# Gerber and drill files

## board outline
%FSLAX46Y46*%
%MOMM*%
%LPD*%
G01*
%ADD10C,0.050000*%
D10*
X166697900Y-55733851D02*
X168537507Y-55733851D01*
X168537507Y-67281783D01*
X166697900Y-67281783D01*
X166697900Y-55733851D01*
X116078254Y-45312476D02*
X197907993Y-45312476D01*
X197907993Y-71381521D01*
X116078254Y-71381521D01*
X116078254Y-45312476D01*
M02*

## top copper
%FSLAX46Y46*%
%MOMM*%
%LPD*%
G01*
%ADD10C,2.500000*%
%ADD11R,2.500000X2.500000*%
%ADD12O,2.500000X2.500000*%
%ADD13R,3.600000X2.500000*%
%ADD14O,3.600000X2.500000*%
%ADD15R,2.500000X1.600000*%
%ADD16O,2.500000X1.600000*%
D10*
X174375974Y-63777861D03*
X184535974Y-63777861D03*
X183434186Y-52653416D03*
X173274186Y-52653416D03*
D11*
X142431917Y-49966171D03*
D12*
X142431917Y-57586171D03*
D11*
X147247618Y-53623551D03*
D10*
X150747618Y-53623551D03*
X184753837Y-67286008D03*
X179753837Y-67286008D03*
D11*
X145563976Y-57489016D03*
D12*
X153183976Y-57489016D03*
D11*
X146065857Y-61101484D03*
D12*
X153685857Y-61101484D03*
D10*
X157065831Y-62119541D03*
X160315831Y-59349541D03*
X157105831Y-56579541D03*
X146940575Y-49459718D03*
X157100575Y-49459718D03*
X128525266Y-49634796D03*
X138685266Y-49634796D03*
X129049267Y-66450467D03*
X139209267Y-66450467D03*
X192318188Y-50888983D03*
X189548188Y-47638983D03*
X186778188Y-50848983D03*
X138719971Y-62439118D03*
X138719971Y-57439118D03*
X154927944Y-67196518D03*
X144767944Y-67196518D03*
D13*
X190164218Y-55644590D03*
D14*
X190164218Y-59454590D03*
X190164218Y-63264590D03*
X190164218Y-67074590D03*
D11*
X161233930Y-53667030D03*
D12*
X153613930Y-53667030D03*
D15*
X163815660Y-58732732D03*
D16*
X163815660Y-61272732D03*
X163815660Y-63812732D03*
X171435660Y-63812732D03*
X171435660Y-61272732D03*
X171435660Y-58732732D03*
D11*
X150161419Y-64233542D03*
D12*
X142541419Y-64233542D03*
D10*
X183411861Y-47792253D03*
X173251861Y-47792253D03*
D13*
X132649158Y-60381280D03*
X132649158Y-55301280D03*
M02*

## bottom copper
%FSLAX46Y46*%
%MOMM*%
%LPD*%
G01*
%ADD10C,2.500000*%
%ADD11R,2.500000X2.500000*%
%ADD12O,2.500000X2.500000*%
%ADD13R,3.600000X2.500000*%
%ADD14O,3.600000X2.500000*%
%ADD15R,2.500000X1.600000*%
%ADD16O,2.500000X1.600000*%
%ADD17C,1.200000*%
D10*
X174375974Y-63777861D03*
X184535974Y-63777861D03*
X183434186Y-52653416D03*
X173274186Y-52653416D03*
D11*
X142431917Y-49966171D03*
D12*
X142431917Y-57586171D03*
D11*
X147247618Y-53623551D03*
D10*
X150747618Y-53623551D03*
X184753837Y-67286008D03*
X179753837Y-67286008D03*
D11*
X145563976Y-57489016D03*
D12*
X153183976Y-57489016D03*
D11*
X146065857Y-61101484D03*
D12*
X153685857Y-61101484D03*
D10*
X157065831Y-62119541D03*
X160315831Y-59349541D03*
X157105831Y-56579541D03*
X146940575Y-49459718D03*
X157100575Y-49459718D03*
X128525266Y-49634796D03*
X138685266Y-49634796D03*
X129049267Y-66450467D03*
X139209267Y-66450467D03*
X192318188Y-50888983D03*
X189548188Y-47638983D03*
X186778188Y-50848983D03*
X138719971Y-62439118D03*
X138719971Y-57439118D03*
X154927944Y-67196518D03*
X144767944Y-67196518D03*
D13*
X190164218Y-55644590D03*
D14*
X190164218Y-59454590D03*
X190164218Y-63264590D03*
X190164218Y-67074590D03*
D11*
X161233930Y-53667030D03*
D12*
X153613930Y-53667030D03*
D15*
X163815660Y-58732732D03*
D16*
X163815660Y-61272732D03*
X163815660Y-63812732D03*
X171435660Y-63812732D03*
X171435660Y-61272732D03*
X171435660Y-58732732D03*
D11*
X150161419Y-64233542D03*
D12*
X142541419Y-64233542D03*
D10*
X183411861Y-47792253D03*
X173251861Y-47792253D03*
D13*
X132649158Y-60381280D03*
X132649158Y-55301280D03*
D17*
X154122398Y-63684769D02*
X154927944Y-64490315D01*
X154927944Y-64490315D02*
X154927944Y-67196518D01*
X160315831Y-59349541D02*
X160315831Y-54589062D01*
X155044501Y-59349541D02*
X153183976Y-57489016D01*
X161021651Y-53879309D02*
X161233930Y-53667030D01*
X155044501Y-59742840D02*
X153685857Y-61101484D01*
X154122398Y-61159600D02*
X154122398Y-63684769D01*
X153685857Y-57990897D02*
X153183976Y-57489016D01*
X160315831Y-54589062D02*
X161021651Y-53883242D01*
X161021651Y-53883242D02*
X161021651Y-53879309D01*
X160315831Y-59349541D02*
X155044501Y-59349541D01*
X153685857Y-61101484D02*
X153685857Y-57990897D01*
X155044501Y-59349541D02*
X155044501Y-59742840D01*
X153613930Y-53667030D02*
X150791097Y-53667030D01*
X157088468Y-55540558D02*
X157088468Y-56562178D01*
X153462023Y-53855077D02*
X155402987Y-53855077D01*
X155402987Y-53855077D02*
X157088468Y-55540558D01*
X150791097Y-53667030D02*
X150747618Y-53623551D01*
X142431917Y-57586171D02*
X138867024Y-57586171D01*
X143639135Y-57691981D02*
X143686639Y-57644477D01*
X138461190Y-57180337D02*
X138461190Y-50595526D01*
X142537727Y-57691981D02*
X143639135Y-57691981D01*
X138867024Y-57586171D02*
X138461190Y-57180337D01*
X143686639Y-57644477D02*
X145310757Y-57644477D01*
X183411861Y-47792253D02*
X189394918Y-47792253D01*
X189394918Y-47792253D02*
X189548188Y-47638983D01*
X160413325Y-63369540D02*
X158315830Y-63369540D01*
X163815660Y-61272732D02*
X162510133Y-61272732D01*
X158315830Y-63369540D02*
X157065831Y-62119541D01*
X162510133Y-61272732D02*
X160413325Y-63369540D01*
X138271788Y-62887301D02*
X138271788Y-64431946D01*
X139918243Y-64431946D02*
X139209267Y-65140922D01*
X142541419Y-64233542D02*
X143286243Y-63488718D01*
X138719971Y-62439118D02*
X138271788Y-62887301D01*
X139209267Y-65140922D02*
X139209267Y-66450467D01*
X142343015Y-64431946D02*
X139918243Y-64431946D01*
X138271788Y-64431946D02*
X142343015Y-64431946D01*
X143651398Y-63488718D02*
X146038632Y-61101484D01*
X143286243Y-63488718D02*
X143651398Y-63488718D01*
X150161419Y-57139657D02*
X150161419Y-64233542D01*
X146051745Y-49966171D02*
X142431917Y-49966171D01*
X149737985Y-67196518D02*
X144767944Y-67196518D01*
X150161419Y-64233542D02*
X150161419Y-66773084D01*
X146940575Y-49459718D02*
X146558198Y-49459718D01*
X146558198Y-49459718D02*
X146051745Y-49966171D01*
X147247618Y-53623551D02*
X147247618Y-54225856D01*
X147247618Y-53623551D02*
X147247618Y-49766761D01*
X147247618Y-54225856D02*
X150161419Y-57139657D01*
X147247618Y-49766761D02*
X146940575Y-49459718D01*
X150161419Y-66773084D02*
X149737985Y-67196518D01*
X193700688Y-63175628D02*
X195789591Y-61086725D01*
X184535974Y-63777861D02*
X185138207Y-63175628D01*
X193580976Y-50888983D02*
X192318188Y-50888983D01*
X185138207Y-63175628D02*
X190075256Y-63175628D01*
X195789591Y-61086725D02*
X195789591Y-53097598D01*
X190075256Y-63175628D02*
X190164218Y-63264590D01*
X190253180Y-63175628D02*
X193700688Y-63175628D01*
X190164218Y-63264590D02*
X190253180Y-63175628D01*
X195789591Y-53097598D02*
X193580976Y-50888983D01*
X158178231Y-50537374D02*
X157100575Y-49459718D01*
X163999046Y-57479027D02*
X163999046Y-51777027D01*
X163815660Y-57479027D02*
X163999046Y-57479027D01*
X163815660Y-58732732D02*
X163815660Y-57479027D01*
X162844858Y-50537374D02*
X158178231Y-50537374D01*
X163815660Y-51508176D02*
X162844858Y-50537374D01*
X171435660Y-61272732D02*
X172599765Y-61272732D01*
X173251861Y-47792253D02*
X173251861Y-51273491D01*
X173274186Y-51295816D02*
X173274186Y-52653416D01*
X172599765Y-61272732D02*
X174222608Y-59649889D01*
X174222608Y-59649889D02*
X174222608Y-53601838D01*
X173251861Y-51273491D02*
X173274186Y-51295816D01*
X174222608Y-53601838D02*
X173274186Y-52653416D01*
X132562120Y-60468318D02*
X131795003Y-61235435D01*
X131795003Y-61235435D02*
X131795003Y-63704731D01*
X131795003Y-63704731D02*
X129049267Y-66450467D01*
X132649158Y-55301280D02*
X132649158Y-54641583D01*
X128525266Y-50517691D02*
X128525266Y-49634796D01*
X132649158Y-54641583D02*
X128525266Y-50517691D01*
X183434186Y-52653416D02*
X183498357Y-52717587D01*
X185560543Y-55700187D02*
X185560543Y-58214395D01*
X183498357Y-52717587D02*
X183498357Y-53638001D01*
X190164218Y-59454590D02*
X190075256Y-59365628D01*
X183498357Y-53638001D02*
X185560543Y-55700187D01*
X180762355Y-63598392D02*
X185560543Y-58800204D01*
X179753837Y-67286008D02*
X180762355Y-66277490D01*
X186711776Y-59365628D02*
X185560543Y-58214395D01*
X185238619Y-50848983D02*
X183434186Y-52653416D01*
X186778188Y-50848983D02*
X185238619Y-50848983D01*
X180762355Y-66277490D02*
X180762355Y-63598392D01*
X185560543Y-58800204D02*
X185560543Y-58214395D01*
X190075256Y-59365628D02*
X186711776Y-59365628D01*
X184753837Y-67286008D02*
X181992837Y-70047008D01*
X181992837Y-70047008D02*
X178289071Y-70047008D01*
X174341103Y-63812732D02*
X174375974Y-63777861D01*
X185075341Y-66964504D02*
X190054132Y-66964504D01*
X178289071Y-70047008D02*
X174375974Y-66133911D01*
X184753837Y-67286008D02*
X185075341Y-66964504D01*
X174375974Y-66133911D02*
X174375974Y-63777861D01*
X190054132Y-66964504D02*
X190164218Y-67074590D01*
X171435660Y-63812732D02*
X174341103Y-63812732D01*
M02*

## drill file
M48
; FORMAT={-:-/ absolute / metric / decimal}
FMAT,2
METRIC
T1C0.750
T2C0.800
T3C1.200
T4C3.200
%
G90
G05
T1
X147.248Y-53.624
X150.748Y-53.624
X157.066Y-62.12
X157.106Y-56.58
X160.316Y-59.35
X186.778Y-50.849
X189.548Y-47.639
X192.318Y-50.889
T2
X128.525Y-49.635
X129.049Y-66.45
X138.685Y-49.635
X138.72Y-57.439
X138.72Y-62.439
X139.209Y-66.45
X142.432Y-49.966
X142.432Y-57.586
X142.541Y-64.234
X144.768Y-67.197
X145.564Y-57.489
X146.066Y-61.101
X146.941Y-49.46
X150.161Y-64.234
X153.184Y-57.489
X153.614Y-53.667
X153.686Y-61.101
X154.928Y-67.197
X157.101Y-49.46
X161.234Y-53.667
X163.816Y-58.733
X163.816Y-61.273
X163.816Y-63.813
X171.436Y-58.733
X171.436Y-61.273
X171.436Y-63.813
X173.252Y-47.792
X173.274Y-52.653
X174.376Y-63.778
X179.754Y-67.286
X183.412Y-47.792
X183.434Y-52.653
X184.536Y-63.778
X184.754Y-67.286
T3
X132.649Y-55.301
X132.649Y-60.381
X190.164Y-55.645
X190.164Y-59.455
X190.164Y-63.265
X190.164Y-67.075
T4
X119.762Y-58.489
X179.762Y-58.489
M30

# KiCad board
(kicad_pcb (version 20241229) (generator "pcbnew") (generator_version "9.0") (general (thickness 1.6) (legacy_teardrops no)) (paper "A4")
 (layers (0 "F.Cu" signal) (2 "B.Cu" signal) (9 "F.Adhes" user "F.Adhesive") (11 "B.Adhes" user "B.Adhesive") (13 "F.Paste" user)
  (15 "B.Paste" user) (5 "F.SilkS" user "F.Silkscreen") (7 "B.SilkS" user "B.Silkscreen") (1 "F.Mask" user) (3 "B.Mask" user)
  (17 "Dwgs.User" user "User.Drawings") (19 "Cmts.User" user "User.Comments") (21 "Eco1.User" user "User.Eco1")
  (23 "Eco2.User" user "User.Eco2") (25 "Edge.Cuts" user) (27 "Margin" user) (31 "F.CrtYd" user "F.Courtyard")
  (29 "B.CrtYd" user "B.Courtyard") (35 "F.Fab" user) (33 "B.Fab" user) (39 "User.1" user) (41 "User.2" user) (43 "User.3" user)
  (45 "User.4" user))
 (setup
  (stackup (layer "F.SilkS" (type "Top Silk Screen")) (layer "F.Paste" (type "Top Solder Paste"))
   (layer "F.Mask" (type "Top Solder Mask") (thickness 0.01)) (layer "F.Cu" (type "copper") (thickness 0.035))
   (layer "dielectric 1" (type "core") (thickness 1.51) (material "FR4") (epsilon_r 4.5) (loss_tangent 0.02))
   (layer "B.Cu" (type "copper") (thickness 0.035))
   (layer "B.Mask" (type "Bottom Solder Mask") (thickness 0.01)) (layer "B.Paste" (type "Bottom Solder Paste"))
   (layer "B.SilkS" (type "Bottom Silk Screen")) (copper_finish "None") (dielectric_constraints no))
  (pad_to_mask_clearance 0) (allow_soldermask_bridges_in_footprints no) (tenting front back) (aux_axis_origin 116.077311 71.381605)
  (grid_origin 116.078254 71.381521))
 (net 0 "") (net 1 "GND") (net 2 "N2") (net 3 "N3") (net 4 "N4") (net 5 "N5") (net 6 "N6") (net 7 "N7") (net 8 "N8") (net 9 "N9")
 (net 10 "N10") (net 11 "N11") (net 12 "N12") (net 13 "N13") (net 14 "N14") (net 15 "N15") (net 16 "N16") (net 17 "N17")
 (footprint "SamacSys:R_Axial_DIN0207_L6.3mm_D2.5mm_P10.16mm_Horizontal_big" (layer "F.Cu") (at 174.375974 63.777861)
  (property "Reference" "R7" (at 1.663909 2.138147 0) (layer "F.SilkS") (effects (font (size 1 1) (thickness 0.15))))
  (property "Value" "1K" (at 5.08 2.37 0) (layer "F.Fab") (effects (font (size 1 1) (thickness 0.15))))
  (pad "1" thru_hole circle (at 0 0) (size 2.5 2.5) (drill 0.8) (layers "*.Cu" "*.Mask") (remove_unused_layers no) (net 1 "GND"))
  (pad "2" thru_hole circle (at 10.16 0) (size 2.5 2.5) (drill 0.8) (layers "*.Cu" "*.Mask") (remove_unused_layers no) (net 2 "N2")))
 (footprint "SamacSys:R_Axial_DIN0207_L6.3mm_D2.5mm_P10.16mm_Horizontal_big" (layer "F.Cu") (at 183.434186 52.653416 180)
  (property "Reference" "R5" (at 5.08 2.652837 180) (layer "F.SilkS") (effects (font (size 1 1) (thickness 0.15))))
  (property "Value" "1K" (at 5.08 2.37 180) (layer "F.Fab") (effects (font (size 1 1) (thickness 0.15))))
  (pad "1" thru_hole circle (at 0 0 180) (size 2.5 2.5) (drill 0.8) (layers "*.Cu" "*.Mask") (remove_unused_layers no) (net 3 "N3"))
  (pad "2" thru_hole circle (at 10.16 0 180) (size 2.5 2.5) (drill 0.8) (layers "*.Cu" "*.Mask") (remove_unused_layers no) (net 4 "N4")))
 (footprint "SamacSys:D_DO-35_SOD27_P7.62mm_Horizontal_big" (layer "F.Cu") (at 142.431917 49.966171 -90)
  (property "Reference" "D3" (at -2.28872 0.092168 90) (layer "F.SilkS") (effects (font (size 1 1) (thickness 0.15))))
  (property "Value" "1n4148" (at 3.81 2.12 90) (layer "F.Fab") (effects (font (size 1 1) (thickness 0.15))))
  (pad "1" thru_hole rect (at 0 0 270) (size 2.5 2.5) (drill 0.8) (layers "*.Cu" "*.Mask") (remove_unused_layers no) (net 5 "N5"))
  (pad "2" thru_hole oval (at 7.62 0 270) (size 2.5 2.5) (drill 0.8) (layers "*.Cu" "*.Mask") (remove_unused_layers no) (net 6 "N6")))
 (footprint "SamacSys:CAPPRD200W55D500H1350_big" (layer "F.Cu") (at 147.247618 53.623551)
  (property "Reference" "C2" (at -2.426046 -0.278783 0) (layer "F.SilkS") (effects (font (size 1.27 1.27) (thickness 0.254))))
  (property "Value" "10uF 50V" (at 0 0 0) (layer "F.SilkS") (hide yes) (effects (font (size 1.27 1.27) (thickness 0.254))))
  (pad "1" thru_hole rect (at 0 0) (size 2.5 2.5) (drill 0.75) (layers "*.Cu" "*.Mask") (remove_unused_layers no) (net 5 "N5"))
  (pad "2" thru_hole circle (at 3.5 0) (size 2.5 2.5) (drill 0.75) (layers "*.Cu" "*.Mask") (remove_unused_layers no) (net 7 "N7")))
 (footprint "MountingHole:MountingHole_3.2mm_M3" (layer "F.Cu") (at 179.762141 58.489223)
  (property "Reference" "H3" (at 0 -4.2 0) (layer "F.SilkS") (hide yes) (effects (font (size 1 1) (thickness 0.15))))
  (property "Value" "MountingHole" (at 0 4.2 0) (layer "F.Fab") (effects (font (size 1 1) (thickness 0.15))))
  (pad "" np_thru_hole circle (at 0 0) (size 3.2 3.2) (drill 3.2) (layers "*.Cu" "*.Mask")))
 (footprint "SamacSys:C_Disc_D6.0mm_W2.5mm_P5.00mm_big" (layer "F.Cu") (at 184.753837 67.286008 180)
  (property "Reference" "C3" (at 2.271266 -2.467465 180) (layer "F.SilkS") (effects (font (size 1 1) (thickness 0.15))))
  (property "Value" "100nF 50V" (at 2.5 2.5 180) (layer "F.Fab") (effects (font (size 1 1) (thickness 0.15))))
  (pad "1" thru_hole circle (at 0 0 180) (size 2.5 2.5) (drill 0.8) (layers "*.Cu" "*.Mask") (remove_unused_layers no) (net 1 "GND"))
  (pad "2" thru_hole circle (at 5 0 180) (size 2.5 2.5) (drill 0.8) (layers "*.Cu" "*.Mask") (remove_unused_layers no) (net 3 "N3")))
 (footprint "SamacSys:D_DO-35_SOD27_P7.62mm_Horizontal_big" (layer "F.Cu") (at 145.563976 57.489016)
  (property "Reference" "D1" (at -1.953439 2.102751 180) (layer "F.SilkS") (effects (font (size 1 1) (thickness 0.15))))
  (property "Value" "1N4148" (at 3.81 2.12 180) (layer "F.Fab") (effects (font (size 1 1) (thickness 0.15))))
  (pad "1" thru_hole rect (at 0 0) (size 2.5 2.5) (drill 0.8) (layers "*.Cu" "*.Mask") (remove_unused_layers no) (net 6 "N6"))
  (pad "2" thru_hole oval (at 7.62 0) (size 2.5 2.5) (drill 0.8) (layers "*.Cu" "*.Mask") (remove_unused_layers no) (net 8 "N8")))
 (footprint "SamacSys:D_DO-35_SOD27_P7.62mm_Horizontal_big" (layer "F.Cu") (at 146.065857 61.101484)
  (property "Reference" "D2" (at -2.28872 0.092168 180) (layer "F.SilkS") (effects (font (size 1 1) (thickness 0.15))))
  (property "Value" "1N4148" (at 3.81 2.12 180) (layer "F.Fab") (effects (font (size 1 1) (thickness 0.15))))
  (pad "1" thru_hole rect (at 0 0) (size 2.5 2.5) (drill 0.8) (layers "*.Cu" "*.Mask") (remove_unused_layers no) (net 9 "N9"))
  (pad "2" thru_hole oval (at 7.62 0) (size 2.5 2.5) (drill 0.8) (layers "*.Cu" "*.Mask") (remove_unused_layers no) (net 8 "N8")))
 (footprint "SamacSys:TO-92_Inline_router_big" (layer "F.Cu") (at 158.935831 60.659541 90)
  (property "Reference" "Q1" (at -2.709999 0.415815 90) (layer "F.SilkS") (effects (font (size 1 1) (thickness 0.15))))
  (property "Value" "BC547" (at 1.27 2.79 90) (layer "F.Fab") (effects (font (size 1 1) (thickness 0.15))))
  (pad "1" thru_hole circle (at -1.46 -1.87 90) (size 2.5 2.5) (drill 0.75) (layers "*.Cu" "*.Mask") (remove_unused_layers no)
   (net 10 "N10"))
  (pad "2" thru_hole circle (at 1.31 1.38 180) (size 2.5 2.5) (drill 0.75) (layers "*.Cu" "*.Mask") (remove_unused_layers no) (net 8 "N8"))
  (pad "3" thru_hole circle (at 4.08 -1.83 90) (size 2.5 2.5) (drill 0.75) (layers "*.Cu" "*.Mask") (remove_unused_layers no) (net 7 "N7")))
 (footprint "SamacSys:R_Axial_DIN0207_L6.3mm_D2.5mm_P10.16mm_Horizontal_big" (layer "F.Cu") (at 146.940575 49.459718)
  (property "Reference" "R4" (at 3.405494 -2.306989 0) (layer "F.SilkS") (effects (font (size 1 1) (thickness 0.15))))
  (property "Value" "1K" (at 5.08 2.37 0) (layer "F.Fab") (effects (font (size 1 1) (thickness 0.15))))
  (pad "1" thru_hole circle (at 0 0) (size 2.5 2.5) (drill 0.8) (layers "*.Cu" "*.Mask") (remove_unused_layers no) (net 5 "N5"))
  (pad "2" thru_hole circle (at 10.16 0) (size 2.5 2.5) (drill 0.8) (layers "*.Cu" "*.Mask") (remove_unused_layers no) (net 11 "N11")))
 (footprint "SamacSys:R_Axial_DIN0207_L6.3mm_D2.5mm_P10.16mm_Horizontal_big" (layer "F.Cu") (at 128.525266 49.634796)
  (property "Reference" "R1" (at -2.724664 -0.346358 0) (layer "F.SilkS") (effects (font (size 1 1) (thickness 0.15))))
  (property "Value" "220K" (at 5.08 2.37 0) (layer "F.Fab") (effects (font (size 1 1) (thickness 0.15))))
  (pad "1" thru_hole circle (at 0 0) (size 2.5 2.5) (drill 0.8) (layers "*.Cu" "*.Mask") (remove_unused_layers no) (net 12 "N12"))
  (pad "2" thru_hole circle (at 10.16 0) (size 2.5 2.5) (drill 0.8) (layers "*.Cu" "*.Mask") (remove_unused_layers no) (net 6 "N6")))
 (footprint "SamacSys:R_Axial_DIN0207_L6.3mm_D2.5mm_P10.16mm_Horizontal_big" (layer "F.Cu") (at 129.049267 66.450467)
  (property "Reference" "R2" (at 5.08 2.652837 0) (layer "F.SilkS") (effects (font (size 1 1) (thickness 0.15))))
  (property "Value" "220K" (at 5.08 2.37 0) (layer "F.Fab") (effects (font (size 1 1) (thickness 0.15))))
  (pad "1" thru_hole circle (at 0 0) (size 2.5 2.5) (drill 0.8) (layers "*.Cu" "*.Mask") (remove_unused_layers no) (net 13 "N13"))
  (pad "2" thru_hole circle (at 10.16 0) (size 2.5 2.5) (drill 0.8) (layers "*.Cu" "*.Mask") (remove_unused_layers no) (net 9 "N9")))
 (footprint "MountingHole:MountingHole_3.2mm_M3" (layer "F.Cu") (at 119.762141 58.489223)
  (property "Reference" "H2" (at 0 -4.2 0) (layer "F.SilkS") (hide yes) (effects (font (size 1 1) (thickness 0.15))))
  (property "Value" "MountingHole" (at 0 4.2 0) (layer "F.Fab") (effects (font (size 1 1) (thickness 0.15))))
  (pad "" np_thru_hole circle (at 0 0) (size 3.2 3.2) (drill 3.2) (layers "*.Cu" "*.Mask")))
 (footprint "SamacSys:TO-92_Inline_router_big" (layer "F.Cu") (at 190.858188 49.018983 180)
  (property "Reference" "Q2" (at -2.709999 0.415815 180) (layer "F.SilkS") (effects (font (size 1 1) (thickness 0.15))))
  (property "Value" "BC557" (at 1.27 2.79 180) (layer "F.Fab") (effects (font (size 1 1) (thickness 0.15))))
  (pad "1" thru_hole circle (at -1.46 -1.87 180) (size 2.5 2.5) (drill 0.75) (layers "*.Cu" "*.Mask") (remove_unused_layers no) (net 2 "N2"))
  (pad "2" thru_hole circle (at 1.31 1.38 270) (size 2.5 2.5) (drill 0.75) (layers "*.Cu" "*.Mask") (remove_unused_layers no) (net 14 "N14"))
  (pad "3" thru_hole circle (at 4.08 -1.83 180) (size 2.5 2.5) (drill 0.75) (layers "*.Cu" "*.Mask") (remove_unused_layers no) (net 3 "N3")))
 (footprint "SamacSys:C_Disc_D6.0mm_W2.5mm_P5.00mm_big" (layer "F.Cu") (at 138.719971 62.439118 90)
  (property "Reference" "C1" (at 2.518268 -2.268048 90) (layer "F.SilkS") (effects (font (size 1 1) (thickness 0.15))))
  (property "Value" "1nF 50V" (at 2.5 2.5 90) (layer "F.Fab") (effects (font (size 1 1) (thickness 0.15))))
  (pad "1" thru_hole circle (at 0 0 90) (size 2.5 2.5) (drill 0.8) (layers "*.Cu" "*.Mask") (remove_unused_layers no) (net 9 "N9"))
  (pad "2" thru_hole circle (at 5 0 90) (size 2.5 2.5) (drill 0.8) (layers "*.Cu" "*.Mask") (remove_unused_layers no) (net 6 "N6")))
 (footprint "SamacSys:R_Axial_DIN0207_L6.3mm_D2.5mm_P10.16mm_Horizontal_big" (layer "F.Cu") (at 154.927944 67.196518 180)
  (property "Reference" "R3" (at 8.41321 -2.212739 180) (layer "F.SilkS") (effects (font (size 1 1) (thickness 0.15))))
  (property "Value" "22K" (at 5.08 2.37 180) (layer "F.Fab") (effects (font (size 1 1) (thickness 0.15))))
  (pad "1" thru_hole circle (at 0 0 180) (size 2.5 2.5) (drill 0.8) (layers "*.Cu" "*.Mask") (remove_unused_layers no) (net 8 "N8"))
  (pad "2" thru_hole circle (at 10.16 0 180) (size 2.5 2.5) (drill 0.8) (layers "*.Cu" "*.Mask") (remove_unused_layers no) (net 5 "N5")))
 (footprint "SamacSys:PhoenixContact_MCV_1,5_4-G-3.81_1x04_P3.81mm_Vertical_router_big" (layer "F.Cu") (at 190.164218 55.64459 -90)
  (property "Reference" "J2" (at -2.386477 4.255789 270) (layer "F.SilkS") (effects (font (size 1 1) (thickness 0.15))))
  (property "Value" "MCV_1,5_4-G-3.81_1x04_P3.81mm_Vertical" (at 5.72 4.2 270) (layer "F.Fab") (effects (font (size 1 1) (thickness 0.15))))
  (pad "1" thru_hole rect (at 0 0 270) (size 2.5 3.6) (drill 1.2) (layers "*.Cu" "*.Mask") (remove_unused_layers no) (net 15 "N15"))
  (pad "2" thru_hole oval (at 3.81 0 270) (size 2.5 3.6) (drill 1.2) (layers "*.Cu" "*.Mask") (remove_unused_layers no) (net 3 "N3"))
  (pad "3" thru_hole oval (at 7.62 0 270) (size 2.5 3.6) (drill 1.2) (layers "*.Cu" "*.Mask") (remove_unused_layers no) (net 2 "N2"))
  (pad "4" thru_hole oval (at 11.43 0 270) (size 2.5 3.6) (drill 1.2) (layers "*.Cu" "*.Mask") (remove_unused_layers no) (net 1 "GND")))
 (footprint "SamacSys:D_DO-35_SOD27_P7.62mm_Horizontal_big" (layer "F.Cu") (at 161.23393 53.66703 180)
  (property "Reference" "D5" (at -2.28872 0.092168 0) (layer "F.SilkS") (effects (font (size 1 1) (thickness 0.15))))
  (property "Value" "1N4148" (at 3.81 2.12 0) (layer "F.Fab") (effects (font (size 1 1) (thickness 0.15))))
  (pad "1" thru_hole rect (at 0 0 180) (size 2.5 2.5) (drill 0.8) (layers "*.Cu" "*.Mask") (remove_unused_layers no) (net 8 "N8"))
  (pad "2" thru_hole oval (at 7.62 0 180) (size 2.5 2.5) (drill 0.8) (layers "*.Cu" "*.Mask") (remove_unused_layers no) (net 7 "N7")))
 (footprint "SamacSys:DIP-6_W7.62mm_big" (layer "F.Cu") (at 163.81566 58.732732)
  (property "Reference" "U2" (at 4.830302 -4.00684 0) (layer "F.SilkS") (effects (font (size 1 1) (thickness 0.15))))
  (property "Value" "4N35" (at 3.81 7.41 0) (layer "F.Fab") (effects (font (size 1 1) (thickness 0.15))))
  (pad "1" thru_hole rect (at 0 0) (size 2.5 1.6) (drill 0.8) (layers "*.Cu" "*.Mask") (remove_unused_layers no) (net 11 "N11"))
  (pad "2" thru_hole oval (at 0 2.54) (size 2.5 1.6) (drill 0.8) (layers "*.Cu" "*.Mask") (remove_unused_layers no) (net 10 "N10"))
  (pad "3" thru_hole oval (at 0 5.08) (size 2.5 1.6) (drill 0.8) (layers "*.Cu" "*.Mask") (remove_unused_layers no) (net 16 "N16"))
  (pad "4" thru_hole oval (at 7.62 5.08) (size 2.5 1.6) (drill 0.8) (layers "*.Cu" "*.Mask") (remove_unused_layers no) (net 1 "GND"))
  (pad "5" thru_hole oval (at 7.62 2.54) (size 2.5 1.6) (drill 0.8) (layers "*.Cu" "*.Mask") (remove_unused_layers no) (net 4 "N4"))
  (pad "6" thru_hole oval (at 7.62 0) (size 2.5 1.6) (drill 0.8) (layers "*.Cu" "*.Mask") (remove_unused_layers no) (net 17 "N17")))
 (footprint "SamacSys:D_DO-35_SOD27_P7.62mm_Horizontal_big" (layer "F.Cu") (at 150.161419 64.233542 180)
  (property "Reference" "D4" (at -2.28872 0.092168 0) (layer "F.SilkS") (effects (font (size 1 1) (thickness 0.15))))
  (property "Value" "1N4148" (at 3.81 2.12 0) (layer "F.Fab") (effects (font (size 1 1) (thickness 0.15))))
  (pad "1" thru_hole rect (at 0 0 180) (size 2.5 2.5) (drill 0.8) (layers "*.Cu" "*.Mask") (remove_unused_layers no) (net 5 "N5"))
  (pad "2" thru_hole oval (at 7.62 0 180) (size 2.5 2.5) (drill 0.8) (layers "*.Cu" "*.Mask") (remove_unused_layers no) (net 9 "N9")))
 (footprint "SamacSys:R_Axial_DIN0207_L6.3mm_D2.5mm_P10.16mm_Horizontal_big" (layer "F.Cu") (at 183.411861 47.792253 180)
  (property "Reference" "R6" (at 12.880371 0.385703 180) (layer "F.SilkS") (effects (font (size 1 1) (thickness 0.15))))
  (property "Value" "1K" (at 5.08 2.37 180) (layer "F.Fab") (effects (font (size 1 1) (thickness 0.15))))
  (pad "1" thru_hole circle (at 0 0 180) (size 2.5 2.5) (drill 0.8) (layers "*.Cu" "*.Mask") (remove_unused_layers no) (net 14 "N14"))
  (pad "2" thru_hole circle (at 10.16 0 180) (size 2.5 2.5) (drill 0.8) (layers "*.Cu" "*.Mask") (remove_unused_layers no) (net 4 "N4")))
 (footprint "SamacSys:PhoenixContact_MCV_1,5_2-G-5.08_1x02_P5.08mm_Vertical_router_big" (layer "F.Cu") (at 132.649158 60.38128 90)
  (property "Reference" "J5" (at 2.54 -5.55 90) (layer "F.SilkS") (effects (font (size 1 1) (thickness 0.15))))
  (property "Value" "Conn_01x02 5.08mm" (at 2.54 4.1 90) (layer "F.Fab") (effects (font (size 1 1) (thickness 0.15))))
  (pad "1" thru_hole rect (at 0 0 90) (size 2.5 3.6) (drill 1.2) (layers "*.Cu" "*.Mask") (remove_unused_layers no) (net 13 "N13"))
  (pad "2" thru_hole rect (at 5.08 0 90) (size 2.5 3.6) (drill 1.2) (layers "*.Cu" "*.Mask") (remove_unused_layers no) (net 12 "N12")))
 (gr_rect (start 166.6979 55.733851) (end 168.537507 67.281783) (stroke (width 0.05) (type default)) (fill no) (layer "Edge.Cuts"))
 (gr_rect (start 116.078254 45.312476) (end 197.907993 71.381521) (stroke (width 0.05) (type default)) (fill no) (layer "Edge.Cuts"))
 (segment (start 154.122398 63.684769) (end 154.927944 64.490315) (width 1.2) (layer "B.Cu") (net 8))
 (segment (start 154.927944 64.490315) (end 154.927944 67.196518) (width 1.2) (layer "B.Cu") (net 8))
 (segment (start 160.315831 59.349541) (end 160.315831 54.589062) (width 1.2) (layer "B.Cu") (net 8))
 (segment (start 155.044501 59.349541) (end 153.183976 57.489016) (width 1.2) (layer "B.Cu") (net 8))
 (segment (start 161.021651 53.879309) (end 161.23393 53.66703) (width 1.2) (layer "B.Cu") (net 8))
 (segment (start 155.044501 59.74284) (end 153.685857 61.101484) (width 1.2) (layer "B.Cu") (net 8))
 (segment (start 154.122398 61.1596) (end 154.122398 63.684769) (width 1.2) (layer "B.Cu") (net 8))
 (segment (start 153.685857 57.990897) (end 153.183976 57.489016) (width 1.2) (layer "B.Cu") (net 8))
 (segment (start 160.315831 54.589062) (end 161.021651 53.883242) (width 1.2) (layer "B.Cu") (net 8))
 (segment (start 161.021651 53.883242) (end 161.021651 53.879309) (width 1.2) (layer "B.Cu") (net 8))
 (segment (start 160.315831 59.349541) (end 155.044501 59.349541) (width 1.2) (layer "B.Cu") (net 8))
 (segment (start 153.685857 61.101484) (end 153.685857 57.990897) (width 1.2) (layer "B.Cu") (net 8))
 (segment (start 155.044501 59.349541) (end 155.044501 59.74284) (width 1.2) (layer "B.Cu") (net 8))
 (segment (start 153.61393 53.66703) (end 150.791097 53.66703) (width 1.2) (layer "B.Cu") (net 7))
 (segment (start 157.088468 55.540558) (end 157.088468 56.562178) (width 1.2) (layer "B.Cu") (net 7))
 (segment (start 153.462023 53.855077) (end 155.402987 53.855077) (width 1.2) (layer "B.Cu") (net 7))
 (segment (start 155.402987 53.855077) (end 157.088468 55.540558) (width 1.2) (layer "B.Cu") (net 7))
 (segment (start 150.791097 53.66703) (end 150.747618 53.623551) (width 1.2) (layer "B.Cu") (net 7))
 (segment (start 142.431917 57.586171) (end 138.867024 57.586171) (width 1.2) (layer "B.Cu") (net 6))
 (segment (start 143.639135 57.691981) (end 143.686639 57.644477) (width 1.2) (layer "B.Cu") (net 6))
 (segment (start 138.46119 57.180337) (end 138.46119 50.595526) (width 1.2) (layer "B.Cu") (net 6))
 (segment (start 142.537727 57.691981) (end 143.639135 57.691981) (width 1.2) (layer "B.Cu") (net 6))
 (segment (start 138.867024 57.586171) (end 138.46119 57.180337) (width 1.2) (layer "B.Cu") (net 6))
 (segment (start 143.686639 57.644477) (end 145.310757 57.644477) (width 1.2) (layer "B.Cu") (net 6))
 (segment (start 183.411861 47.792253) (end 189.394918 47.792253) (width 1.2) (layer "B.Cu") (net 14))
 (segment (start 189.394918 47.792253) (end 189.548188 47.638983) (width 1.2) (layer "B.Cu") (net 14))
 (segment (start 160.413325 63.36954) (end 158.31583 63.36954) (width 1.2) (layer "B.Cu") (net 10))
 (segment (start 163.81566 61.272732) (end 162.510133 61.272732) (width 1.2) (layer "B.Cu") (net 10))
 (segment (start 158.31583 63.36954) (end 157.065831 62.119541) (width 1.2) (layer "B.Cu") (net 10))
 (segment (start 162.510133 61.272732) (end 160.413325 63.36954) (width 1.2) (layer "B.Cu") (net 10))
 (segment (start 138.271788 62.887301) (end 138.271788 64.431946) (width 1.2) (layer "B.Cu") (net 9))
 (segment (start 139.918243 64.431946) (end 139.209267 65.140922) (width 1.2) (layer "B.Cu") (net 9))
 (segment (start 142.541419 64.233542) (end 143.286243 63.488718) (width 1.2) (layer "B.Cu") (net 9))
 (segment (start 138.719971 62.439118) (end 138.271788 62.887301) (width 1.2) (layer "B.Cu") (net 9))
 (segment (start 139.209267 65.140922) (end 139.209267 66.450467) (width 1.2) (layer "B.Cu") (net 9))
 (segment (start 142.343015 64.431946) (end 139.918243 64.431946) (width 1.2) (layer "B.Cu") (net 9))
 (segment (start 138.271788 64.431946) (end 142.343015 64.431946) (width 1.2) (layer "B.Cu") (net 9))
 (segment (start 143.651398 63.488718) (end 146.038632 61.101484) (width 1.2) (layer "B.Cu") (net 9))
 (segment (start 143.286243 63.488718) (end 143.651398 63.488718) (width 1.2) (layer "B.Cu") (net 9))
 (segment (start 150.161419 57.139657) (end 150.161419 64.233542) (width 1.2) (layer "B.Cu") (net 5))
 (segment (start 146.051745 49.966171) (end 142.431917 49.966171) (width 1.2) (layer "B.Cu") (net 5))
 (segment (start 149.737985 67.196518) (end 144.767944 67.196518) (width 1.2) (layer "B.Cu") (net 5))
 (segment (start 150.161419 64.233542) (end 150.161419 66.773084) (width 1.2) (layer "B.Cu") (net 5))
 (segment (start 146.940575 49.459718) (end 146.558198 49.459718) (width 1.2) (layer "B.Cu") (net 5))
 (segment (start 146.558198 49.459718) (end 146.051745 49.966171) (width 1.2) (layer "B.Cu") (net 5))
 (segment (start 147.247618 53.623551) (end 147.247618 54.225856) (width 1.2) (layer "B.Cu") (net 5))
 (segment (start 147.247618 53.623551) (end 147.247618 49.766761) (width 1.2) (layer "B.Cu") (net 5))
 (segment (start 147.247618 54.225856) (end 150.161419 57.139657) (width 1.2) (layer "B.Cu") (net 5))
 (segment (start 147.247618 49.766761) (end 146.940575 49.459718) (width 1.2) (layer "B.Cu") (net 5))
 (segment (start 150.161419 66.773084) (end 149.737985 67.196518) (width 1.2) (layer "B.Cu") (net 5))
 (segment (start 193.700688 63.175628) (end 195.789591 61.086725) (width 1.2) (layer "B.Cu") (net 2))
 (segment (start 184.535974 63.777861) (end 185.138207 63.175628) (width 1.2) (layer "B.Cu") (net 2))
 (segment (start 193.580976 50.888983) (end 192.318188 50.888983) (width 1.2) (layer "B.Cu") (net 2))
 (segment (start 185.138207 63.175628) (end 190.075256 63.175628) (width 1.2) (layer "B.Cu") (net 2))
 (segment (start 195.789591 61.086725) (end 195.789591 53.097598) (width 1.2) (layer "B.Cu") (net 2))
 (segment (start 190.075256 63.175628) (end 190.164218 63.26459) (width 1.2) (layer "B.Cu") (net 2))
 (segment (start 190.25318 63.175628) (end 193.700688 63.175628) (width 1.2) (layer "B.Cu") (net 2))
 (segment (start 190.164218 63.26459) (end 190.25318 63.175628) (width 1.2) (layer "B.Cu") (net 2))
 (segment (start 195.789591 53.097598) (end 193.580976 50.888983) (width 1.2) (layer "B.Cu") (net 2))
 (segment (start 158.178231 50.537374) (end 157.100575 49.459718) (width 1.2) (layer "B.Cu") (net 11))
 (segment (start 163.999046 57.479027) (end 163.999046 51.777027) (width 1.2) (layer "B.Cu") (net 11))
 (segment (start 163.81566 57.479027) (end 163.999046 57.479027) (width 1.2) (layer "B.Cu") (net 11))
 (segment (start 163.81566 58.732732) (end 163.81566 57.479027) (width 1.2) (layer "B.Cu") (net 11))
 (segment (start 162.844858 50.537374) (end 158.178231 50.537374) (width 1.2) (layer "B.Cu") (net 11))
 (segment (start 163.81566 51.508176) (end 162.844858 50.537374) (width 1.2) (layer "B.Cu") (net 11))
 (segment (start 171.43566 61.272732) (end 172.599765 61.272732) (width 1.2) (layer "B.Cu") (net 4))
 (segment (start 173.251861 47.792253) (end 173.251861 51.273491) (width 1.2) (layer "B.Cu") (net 4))
 (segment (start 173.274186 51.295816) (end 173.274186 52.653416) (width 1.2) (layer "B.Cu") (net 4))
 (segment (start 172.599765 61.272732) (end 174.222608 59.649889) (width 1.2) (layer "B.Cu") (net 4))
 (segment (start 174.222608 59.649889) (end 174.222608 53.601838) (width 1.2) (layer "B.Cu") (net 4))
 (segment (start 173.251861 51.273491) (end 173.274186 51.295816) (width 1.2) (layer "B.Cu") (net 4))
 (segment (start 174.222608 53.601838) (end 173.274186 52.653416) (width 1.2) (layer "B.Cu") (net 4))
 (segment (start 132.56212 60.468318) (end 131.795003 61.235435) (width 1.2) (layer "B.Cu") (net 13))
 (segment (start 131.795003 61.235435) (end 131.795003 63.704731) (width 1.2) (layer "B.Cu") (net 13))
 (segment (start 131.795003 63.704731) (end 129.049267 66.450467) (width 1.2) (layer "B.Cu") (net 13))
 (segment (start 132.649158 55.30128) (end 132.649158 54.641583) (width 1.2) (layer "B.Cu") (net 12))
 (segment (start 128.525266 50.517691) (end 128.525266 49.634796) (width 1.2) (layer "B.Cu") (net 12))
 (segment (start 132.649158 54.641583) (end 128.525266 50.517691) (width 1.2) (layer "B.Cu") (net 12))
 (segment (start 183.434186 52.653416) (end 183.498357 52.717587) (width 1.2) (layer "B.Cu") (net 3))
 (segment (start 185.560543 55.700187) (end 185.560543 58.214395) (width 1.2) (layer "B.Cu") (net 3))
 (segment (start 183.498357 52.717587) (end 183.498357 53.638001) (width 1.2) (layer "B.Cu") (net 3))
 (segment (start 190.164218 59.45459) (end 190.075256 59.365628) (width 1.2) (layer "B.Cu") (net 3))
 (segment (start 183.498357 53.638001) (end 185.560543 55.700187) (width 1.2) (layer "B.Cu") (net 3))
 (segment (start 180.762355 63.598392) (end 185.560543 58.800204) (width 1.2) (layer "B.Cu") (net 3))
 (segment (start 179.753837 67.286008) (end 180.762355 66.27749) (width 1.2) (layer "B.Cu") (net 3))
 (segment (start 186.711776 59.365628) (end 185.560543 58.214395) (width 1.2) (layer "B.Cu") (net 3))
 (segment (start 185.238619 50.848983) (end 183.434186 52.653416) (width 1.2) (layer "B.Cu") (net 3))
 (segment (start 186.778188 50.848983) (end 185.238619 50.848983) (width 1.2) (layer "B.Cu") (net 3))
 (segment (start 180.762355 66.27749) (end 180.762355 63.598392) (width 1.2) (layer "B.Cu") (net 3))
 (segment (start 185.560543 58.800204) (end 185.560543 58.214395) (width 1.2) (layer "B.Cu") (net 3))
 (segment (start 190.075256 59.365628) (end 186.711776 59.365628) (width 1.2) (layer "B.Cu") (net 3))
 (segment (start 184.753837 67.286008) (end 181.992837 70.047008) (width 1.2) (layer "B.Cu") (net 1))
 (segment (start 181.992837 70.047008) (end 178.289071 70.047008) (width 1.2) (layer "B.Cu") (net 1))
 (segment (start 174.341103 63.812732) (end 174.375974 63.777861) (width 1.2) (layer "B.Cu") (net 1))
 (segment (start 185.075341 66.964504) (end 190.054132 66.964504) (width 1.2) (layer "B.Cu") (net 1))
 (segment (start 178.289071 70.047008) (end 174.375974 66.133911) (width 1.2) (layer "B.Cu") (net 1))
 (segment (start 184.753837 67.286008) (end 185.075341 66.964504) (width 1.2) (layer "B.Cu") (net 1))
 (segment (start 174.375974 66.133911) (end 174.375974 63.777861) (width 1.2) (layer "B.Cu") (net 1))
 (segment (start 190.054132 66.964504) (end 190.164218 67.07459) (width 1.2) (layer "B.Cu") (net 1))
 (segment (start 171.43566 63.812732) (end 174.341103 63.812732) (width 1.2) (layer "B.Cu") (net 1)))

